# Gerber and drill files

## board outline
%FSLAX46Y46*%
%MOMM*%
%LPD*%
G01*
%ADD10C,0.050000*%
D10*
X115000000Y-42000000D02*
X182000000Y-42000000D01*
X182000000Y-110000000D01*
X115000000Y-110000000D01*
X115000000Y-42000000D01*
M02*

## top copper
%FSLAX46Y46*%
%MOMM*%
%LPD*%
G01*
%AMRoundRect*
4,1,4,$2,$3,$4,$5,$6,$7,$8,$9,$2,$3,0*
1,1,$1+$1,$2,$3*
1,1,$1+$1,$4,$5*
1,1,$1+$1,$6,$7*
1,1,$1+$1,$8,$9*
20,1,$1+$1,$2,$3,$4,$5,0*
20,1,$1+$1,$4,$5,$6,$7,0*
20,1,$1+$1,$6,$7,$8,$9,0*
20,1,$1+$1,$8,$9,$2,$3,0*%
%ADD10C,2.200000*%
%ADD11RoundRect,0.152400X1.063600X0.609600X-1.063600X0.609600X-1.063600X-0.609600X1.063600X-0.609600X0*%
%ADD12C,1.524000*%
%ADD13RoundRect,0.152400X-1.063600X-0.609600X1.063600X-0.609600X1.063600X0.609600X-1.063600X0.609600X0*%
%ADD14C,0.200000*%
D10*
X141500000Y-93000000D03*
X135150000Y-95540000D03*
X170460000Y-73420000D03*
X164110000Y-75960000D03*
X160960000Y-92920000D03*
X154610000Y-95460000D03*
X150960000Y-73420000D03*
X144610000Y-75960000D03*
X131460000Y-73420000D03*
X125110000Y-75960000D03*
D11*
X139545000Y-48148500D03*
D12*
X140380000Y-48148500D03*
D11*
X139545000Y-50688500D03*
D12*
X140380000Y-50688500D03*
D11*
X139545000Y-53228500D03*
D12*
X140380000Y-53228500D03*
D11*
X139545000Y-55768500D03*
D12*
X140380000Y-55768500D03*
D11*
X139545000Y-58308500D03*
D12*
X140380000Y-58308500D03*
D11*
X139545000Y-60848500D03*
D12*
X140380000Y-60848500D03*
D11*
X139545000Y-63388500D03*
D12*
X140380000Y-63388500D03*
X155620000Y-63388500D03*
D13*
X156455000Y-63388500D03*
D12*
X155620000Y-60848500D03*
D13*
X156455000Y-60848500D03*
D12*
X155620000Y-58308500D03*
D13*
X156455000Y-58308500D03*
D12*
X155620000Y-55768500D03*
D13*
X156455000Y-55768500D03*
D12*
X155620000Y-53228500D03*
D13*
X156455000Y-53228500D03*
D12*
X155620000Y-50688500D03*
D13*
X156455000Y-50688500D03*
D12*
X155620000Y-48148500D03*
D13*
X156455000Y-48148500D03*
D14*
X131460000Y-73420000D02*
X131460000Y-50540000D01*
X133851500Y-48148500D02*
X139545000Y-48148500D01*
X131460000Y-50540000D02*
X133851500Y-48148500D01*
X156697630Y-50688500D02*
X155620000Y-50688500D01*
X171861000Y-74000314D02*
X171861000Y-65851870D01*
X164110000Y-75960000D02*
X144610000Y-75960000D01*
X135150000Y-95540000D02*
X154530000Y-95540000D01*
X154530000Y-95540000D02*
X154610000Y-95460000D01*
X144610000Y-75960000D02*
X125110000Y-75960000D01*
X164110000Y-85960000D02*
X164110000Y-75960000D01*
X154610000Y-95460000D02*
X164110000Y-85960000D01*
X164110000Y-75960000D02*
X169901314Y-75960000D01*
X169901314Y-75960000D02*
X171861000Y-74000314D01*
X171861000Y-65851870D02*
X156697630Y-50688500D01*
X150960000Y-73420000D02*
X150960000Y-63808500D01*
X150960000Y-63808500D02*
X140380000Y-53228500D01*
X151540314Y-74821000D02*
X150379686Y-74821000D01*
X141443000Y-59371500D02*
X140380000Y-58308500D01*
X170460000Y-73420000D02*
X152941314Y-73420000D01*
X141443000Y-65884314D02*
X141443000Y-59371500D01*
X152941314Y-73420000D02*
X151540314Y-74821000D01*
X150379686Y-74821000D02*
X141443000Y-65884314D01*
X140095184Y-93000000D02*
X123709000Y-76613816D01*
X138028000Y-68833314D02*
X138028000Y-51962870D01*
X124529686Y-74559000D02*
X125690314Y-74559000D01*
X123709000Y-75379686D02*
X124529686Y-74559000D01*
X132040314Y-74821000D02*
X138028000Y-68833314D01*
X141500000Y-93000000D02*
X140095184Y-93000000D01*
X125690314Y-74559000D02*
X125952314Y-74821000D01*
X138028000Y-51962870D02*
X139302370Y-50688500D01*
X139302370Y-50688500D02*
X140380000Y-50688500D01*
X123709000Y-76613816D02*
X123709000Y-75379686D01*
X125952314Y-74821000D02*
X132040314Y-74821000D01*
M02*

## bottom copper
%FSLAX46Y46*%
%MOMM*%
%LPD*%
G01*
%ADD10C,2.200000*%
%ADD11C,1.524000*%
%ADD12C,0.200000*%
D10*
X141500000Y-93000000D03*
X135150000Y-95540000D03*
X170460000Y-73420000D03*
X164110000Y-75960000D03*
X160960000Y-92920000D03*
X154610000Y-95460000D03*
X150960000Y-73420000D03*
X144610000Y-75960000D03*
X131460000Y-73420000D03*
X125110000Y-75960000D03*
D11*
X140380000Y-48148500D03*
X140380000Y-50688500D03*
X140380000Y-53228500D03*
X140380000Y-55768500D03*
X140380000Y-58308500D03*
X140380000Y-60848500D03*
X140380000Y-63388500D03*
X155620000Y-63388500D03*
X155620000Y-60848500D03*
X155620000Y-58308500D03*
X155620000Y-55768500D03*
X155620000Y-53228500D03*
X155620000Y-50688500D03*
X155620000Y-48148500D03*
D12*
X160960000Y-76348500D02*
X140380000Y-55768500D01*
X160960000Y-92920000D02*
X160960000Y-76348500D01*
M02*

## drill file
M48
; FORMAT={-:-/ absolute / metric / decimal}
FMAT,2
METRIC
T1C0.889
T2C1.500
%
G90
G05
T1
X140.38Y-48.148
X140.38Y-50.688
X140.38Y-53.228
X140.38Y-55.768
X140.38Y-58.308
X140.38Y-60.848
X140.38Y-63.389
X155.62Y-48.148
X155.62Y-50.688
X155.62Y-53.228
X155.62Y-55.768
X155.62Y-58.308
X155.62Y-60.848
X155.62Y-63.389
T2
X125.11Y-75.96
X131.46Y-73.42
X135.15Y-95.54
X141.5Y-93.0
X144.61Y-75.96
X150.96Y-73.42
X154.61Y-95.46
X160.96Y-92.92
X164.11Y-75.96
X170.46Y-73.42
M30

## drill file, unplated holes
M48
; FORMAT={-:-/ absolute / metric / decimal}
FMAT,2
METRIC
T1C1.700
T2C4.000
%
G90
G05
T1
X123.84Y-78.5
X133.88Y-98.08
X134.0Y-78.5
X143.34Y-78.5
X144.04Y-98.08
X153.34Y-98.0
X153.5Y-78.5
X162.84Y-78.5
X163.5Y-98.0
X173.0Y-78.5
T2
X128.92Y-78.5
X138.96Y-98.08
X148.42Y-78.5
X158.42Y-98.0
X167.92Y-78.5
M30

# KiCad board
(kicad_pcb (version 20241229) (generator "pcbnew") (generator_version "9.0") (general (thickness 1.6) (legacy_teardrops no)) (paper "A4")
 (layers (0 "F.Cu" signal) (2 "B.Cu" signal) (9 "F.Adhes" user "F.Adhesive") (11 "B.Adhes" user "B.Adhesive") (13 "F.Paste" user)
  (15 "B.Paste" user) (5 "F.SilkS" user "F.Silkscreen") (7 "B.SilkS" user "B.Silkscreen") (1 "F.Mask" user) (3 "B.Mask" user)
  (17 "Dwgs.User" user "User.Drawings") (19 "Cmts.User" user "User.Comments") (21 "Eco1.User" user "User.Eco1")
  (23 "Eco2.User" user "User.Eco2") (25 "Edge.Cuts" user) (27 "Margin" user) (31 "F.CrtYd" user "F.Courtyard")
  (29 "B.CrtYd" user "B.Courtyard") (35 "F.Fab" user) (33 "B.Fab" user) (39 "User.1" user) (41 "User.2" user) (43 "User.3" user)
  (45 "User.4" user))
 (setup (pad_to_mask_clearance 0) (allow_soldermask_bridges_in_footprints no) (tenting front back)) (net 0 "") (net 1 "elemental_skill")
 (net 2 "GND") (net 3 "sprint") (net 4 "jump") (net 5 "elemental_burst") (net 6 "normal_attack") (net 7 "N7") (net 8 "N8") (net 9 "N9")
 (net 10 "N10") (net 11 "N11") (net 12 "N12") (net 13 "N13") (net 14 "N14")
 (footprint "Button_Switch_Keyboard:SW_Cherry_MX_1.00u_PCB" (layer "F.Cu") (at 141.5 93)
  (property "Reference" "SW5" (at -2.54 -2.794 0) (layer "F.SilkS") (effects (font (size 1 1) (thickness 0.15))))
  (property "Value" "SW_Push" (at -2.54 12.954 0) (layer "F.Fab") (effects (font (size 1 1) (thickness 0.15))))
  (pad "" np_thru_hole circle (at -7.62 5.08) (size 1.7 1.7) (drill 1.7) (layers "*.Cu" "*.Mask"))
  (pad "" np_thru_hole circle (at -2.54 5.08) (size 4 4) (drill 4) (layers "*.Cu" "*.Mask"))
  (pad "" np_thru_hole circle (at 2.54 5.08) (size 1.7 1.7) (drill 1.7) (layers "*.Cu" "*.Mask"))
  (pad "1" thru_hole circle (at 0 0) (size 2.2 2.2) (drill 1.5) (layers "*.Cu" "*.Mask") (remove_unused_layers no) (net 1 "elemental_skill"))
  (pad "2" thru_hole circle (at -6.35 2.54) (size 2.2 2.2) (drill 1.5) (layers "*.Cu" "*.Mask") (remove_unused_layers no) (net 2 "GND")))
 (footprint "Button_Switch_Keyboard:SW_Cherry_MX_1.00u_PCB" (layer "F.Cu") (at 170.46 73.42)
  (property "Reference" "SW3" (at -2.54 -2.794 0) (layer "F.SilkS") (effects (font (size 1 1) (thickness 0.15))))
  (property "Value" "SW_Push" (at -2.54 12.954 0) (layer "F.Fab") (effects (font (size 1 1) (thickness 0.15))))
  (pad "" np_thru_hole circle (at -7.62 5.08) (size 1.7 1.7) (drill 1.7) (layers "*.Cu" "*.Mask"))
  (pad "" np_thru_hole circle (at -2.54 5.08) (size 4 4) (drill 4) (layers "*.Cu" "*.Mask"))
  (pad "" np_thru_hole circle (at 2.54 5.08) (size 1.7 1.7) (drill 1.7) (layers "*.Cu" "*.Mask"))
  (pad "1" thru_hole circle (at 0 0) (size 2.2 2.2) (drill 1.5) (layers "*.Cu" "*.Mask") (remove_unused_layers no) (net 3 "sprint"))
  (pad "2" thru_hole circle (at -6.35 2.54) (size 2.2 2.2) (drill 1.5) (layers "*.Cu" "*.Mask") (remove_unused_layers no) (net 2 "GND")))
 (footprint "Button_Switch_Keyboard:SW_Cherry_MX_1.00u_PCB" (layer "F.Cu") (at 160.96 92.92)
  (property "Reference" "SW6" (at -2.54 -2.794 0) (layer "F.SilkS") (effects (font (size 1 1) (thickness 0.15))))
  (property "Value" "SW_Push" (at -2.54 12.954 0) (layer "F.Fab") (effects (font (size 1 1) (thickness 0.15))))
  (pad "" np_thru_hole circle (at -7.62 5.08) (size 1.7 1.7) (drill 1.7) (layers "*.Cu" "*.Mask"))
  (pad "" np_thru_hole circle (at -2.54 5.08) (size 4 4) (drill 4) (layers "*.Cu" "*.Mask"))
  (pad "" np_thru_hole circle (at 2.54 5.08) (size 1.7 1.7) (drill 1.7) (layers "*.Cu" "*.Mask"))
  (pad "1" thru_hole circle (at 0 0) (size 2.2 2.2) (drill 1.5) (layers "*.Cu" "*.Mask") (remove_unused_layers no) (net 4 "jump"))
  (pad "2" thru_hole circle (at -6.35 2.54) (size 2.2 2.2) (drill 1.5) (layers "*.Cu" "*.Mask") (remove_unused_layers no) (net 2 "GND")))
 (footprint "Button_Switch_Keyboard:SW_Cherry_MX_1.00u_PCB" (layer "F.Cu") (at 150.96 73.42)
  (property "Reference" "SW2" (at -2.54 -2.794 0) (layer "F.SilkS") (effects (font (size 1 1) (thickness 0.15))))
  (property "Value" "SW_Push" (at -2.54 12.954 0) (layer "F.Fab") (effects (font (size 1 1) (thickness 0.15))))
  (pad "" np_thru_hole circle (at -7.62 5.08) (size 1.7 1.7) (drill 1.7) (layers "*.Cu" "*.Mask"))
  (pad "" np_thru_hole circle (at -2.54 5.08) (size 4 4) (drill 4) (layers "*.Cu" "*.Mask"))
  (pad "" np_thru_hole circle (at 2.54 5.08) (size 1.7 1.7) (drill 1.7) (layers "*.Cu" "*.Mask"))
  (pad "1" thru_hole circle (at 0 0) (size 2.2 2.2) (drill 1.5) (layers "*.Cu" "*.Mask") (remove_unused_layers no) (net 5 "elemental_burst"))
  (pad "2" thru_hole circle (at -6.35 2.54) (size 2.2 2.2) (drill 1.5) (layers "*.Cu" "*.Mask") (remove_unused_layers no) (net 2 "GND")))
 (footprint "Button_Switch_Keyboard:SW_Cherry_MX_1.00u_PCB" (layer "F.Cu") (at 131.46 73.42)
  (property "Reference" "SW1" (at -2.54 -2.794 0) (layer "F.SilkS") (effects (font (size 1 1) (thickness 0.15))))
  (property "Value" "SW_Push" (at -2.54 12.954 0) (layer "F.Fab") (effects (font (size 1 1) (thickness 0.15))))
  (pad "" np_thru_hole circle (at -7.62 5.08) (size 1.7 1.7) (drill 1.7) (layers "*.Cu" "*.Mask"))
  (pad "" np_thru_hole circle (at -2.54 5.08) (size 4 4) (drill 4) (layers "*.Cu" "*.Mask"))
  (pad "" np_thru_hole circle (at 2.54 5.08) (size 1.7 1.7) (drill 1.7) (layers "*.Cu" "*.Mask"))
  (pad "1" thru_hole circle (at 0 0) (size 2.2 2.2) (drill 1.5) (layers "*.Cu" "*.Mask") (remove_unused_layers no) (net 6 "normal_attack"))
  (pad "2" thru_hole circle (at -6.35 2.54) (size 2.2 2.2) (drill 1.5) (layers "*.Cu" "*.Mask") (remove_unused_layers no) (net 2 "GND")))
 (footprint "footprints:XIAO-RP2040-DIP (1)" (layer "F.Cu") (at 148 55.7685)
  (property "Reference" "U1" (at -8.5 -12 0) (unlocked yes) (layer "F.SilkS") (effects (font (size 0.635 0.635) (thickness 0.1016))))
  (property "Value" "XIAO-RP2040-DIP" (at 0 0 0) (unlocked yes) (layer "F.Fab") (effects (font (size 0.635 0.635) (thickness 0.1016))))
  (pad "1" smd roundrect (at -8.455 -7.62 180) (size 2.432 1.524) (layers "F.Cu" "F.Mask") (roundrect_rratio 0.1) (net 6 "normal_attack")
   (thermal_bridge_angle 45))
  (pad "1" thru_hole circle (at -7.62 -7.62 180) (size 1.524 1.524) (drill 0.889) (layers "*.Cu" "*.Mask") (remove_unused_layers no)
   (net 6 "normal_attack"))
  (pad "2" smd roundrect (at -8.455 -5.08 180) (size 2.432 1.524) (layers "F.Cu" "F.Mask") (roundrect_rratio 0.1) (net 1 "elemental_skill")
   (thermal_bridge_angle 45))
  (pad "2" thru_hole circle (at -7.62 -5.08 180) (size 1.524 1.524) (drill 0.889) (layers "*.Cu" "*.Mask") (remove_unused_layers no)
   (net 1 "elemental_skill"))
  (pad "3" smd roundrect (at -8.455 -2.54 180) (size 2.432 1.524) (layers "F.Cu" "F.Mask") (roundrect_rratio 0.1) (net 5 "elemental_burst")
   (thermal_bridge_angle 45))
  (pad "3" thru_hole circle (at -7.62 -2.54 180) (size 1.524 1.524) (drill 0.889) (layers "*.Cu" "*.Mask") (remove_unused_layers no)
   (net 5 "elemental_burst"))
  (pad "4" smd roundrect (at -8.455 0 180) (size 2.432 1.524) (layers "F.Cu" "F.Mask") (roundrect_rratio 0.1) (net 4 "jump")
   (thermal_bridge_angle 45))
  (pad "4" thru_hole circle (at -7.62 0 180) (size 1.524 1.524) (drill 0.889) (layers "*.Cu" "*.Mask") (remove_unused_layers no)
   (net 4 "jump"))
  (pad "5" smd roundrect (at -8.455 2.54 180) (size 2.432 1.524) (layers "F.Cu" "F.Mask") (roundrect_rratio 0.1) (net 3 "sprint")
   (thermal_bridge_angle 45))
  (pad "5" thru_hole circle (at -7.62 2.54 180) (size 1.524 1.524) (drill 0.889) (layers "*.Cu" "*.Mask") (remove_unused_layers no)
   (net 3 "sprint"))
  (pad "6" smd roundrect (at -8.455 5.08 180) (size 2.432 1.524) (layers "F.Cu" "F.Mask") (roundrect_rratio 0.1) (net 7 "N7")
   (thermal_bridge_angle 45))
  (pad "6" thru_hole circle (at -7.62 5.08 180) (size 1.524 1.524) (drill 0.889) (layers "*.Cu" "*.Mask") (remove_unused_layers no)
   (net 7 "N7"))
  (pad "7" smd roundrect (at -8.455 7.62 180) (size 2.432 1.524) (layers "F.Cu" "F.Mask") (roundrect_rratio 0.1) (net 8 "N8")
   (thermal_bridge_angle 45))
  (pad "7" thru_hole circle (at -7.62 7.62 180) (size 1.524 1.524) (drill 0.889) (layers "*.Cu" "*.Mask") (remove_unused_layers no)
   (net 8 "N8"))
  (pad "8" thru_hole circle (at 7.62 7.62) (size 1.524 1.524) (drill 0.889) (layers "*.Cu" "*.Mask") (remove_unused_layers no) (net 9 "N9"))
  (pad "8" smd roundrect (at 8.455 7.62) (size 2.432 1.524) (layers "F.Cu" "F.Mask") (roundrect_rratio 0.1) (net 9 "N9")
   (thermal_bridge_angle 45))
  (pad "9" thru_hole circle (at 7.62 5.08) (size 1.524 1.524) (drill 0.889) (layers "*.Cu" "*.Mask") (remove_unused_layers no)
   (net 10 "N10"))
  (pad "9" smd roundrect (at 8.455 5.08) (size 2.432 1.524) (layers "F.Cu" "F.Mask") (roundrect_rratio 0.1) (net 10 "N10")
   (thermal_bridge_angle 45))
  (pad "10" thru_hole circle (at 7.62 2.54) (size 1.524 1.524) (drill 0.889) (layers "*.Cu" "*.Mask") (remove_unused_layers no)
   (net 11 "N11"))
  (pad "10" smd roundrect (at 8.455 2.54) (size 2.432 1.524) (layers "F.Cu" "F.Mask") (roundrect_rratio 0.1) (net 11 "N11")
   (thermal_bridge_angle 45))
  (pad "11" thru_hole circle (at 7.62 0) (size 1.524 1.524) (drill 0.889) (layers "*.Cu" "*.Mask") (remove_unused_layers no) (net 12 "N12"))
  (pad "11" smd roundrect (at 8.455 0) (size 2.432 1.524) (layers "F.Cu" "F.Mask") (roundrect_rratio 0.1) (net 12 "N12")
   (thermal_bridge_angle 45))
  (pad "12" thru_hole circle (at 7.62 -2.54) (size 1.524 1.524) (drill 0.889) (layers "*.Cu" "*.Mask") (remove_unused_layers no)
   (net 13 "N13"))
  (pad "12" smd roundrect (at 8.455 -2.54) (size 2.432 1.524) (layers "F.Cu" "F.Mask") (roundrect_rratio 0.1) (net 13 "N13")
   (thermal_bridge_angle 45))
  (pad "13" thru_hole circle (at 7.62 -5.08) (size 1.524 1.524) (drill 0.889) (layers "*.Cu" "*.Mask") (remove_unused_layers no)
   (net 2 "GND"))
  (pad "13" smd roundrect (at 8.455 -5.08) (size 2.432 1.524) (layers "F.Cu" "F.Mask") (roundrect_rratio 0.1) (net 2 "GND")
   (thermal_bridge_angle 45))
  (pad "14" thru_hole circle (at 7.62 -7.62) (size 1.524 1.524) (drill 0.889) (layers "*.Cu" "*.Mask") (remove_unused_layers no)
   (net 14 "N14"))
  (pad "14" smd roundrect (at 8.455 -7.62) (size 2.432 1.524) (layers "F.Cu" "F.Mask") (roundrect_rratio 0.1) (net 14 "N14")
   (thermal_bridge_angle 45)))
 (gr_rect (start 115 42) (end 182 110) (stroke (width 0.05) (type solid)) (fill no) (layer "Edge.Cuts"))
 (segment (start 131.46 73.42) (end 131.46 50.54) (width 0.2) (layer "F.Cu") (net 6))
 (segment (start 133.8515 48.1485) (end 139.545 48.1485) (width 0.2) (layer "F.Cu") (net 6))
 (segment (start 131.46 50.54) (end 133.8515 48.1485) (width 0.2) (layer "F.Cu") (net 6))
 (segment (start 156.69763 50.6885) (end 155.62 50.6885) (width 0.2) (layer "F.Cu") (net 2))
 (segment (start 171.861 74.000314) (end 171.861 65.85187) (width 0.2) (layer "F.Cu") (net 2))
 (segment (start 164.11 75.96) (end 144.61 75.96) (width 0.2) (layer "F.Cu") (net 2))
 (segment (start 135.15 95.54) (end 154.53 95.54) (width 0.2) (layer "F.Cu") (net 2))
 (segment (start 154.53 95.54) (end 154.61 95.46) (width 0.2) (layer "F.Cu") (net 2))
 (segment (start 144.61 75.96) (end 125.11 75.96) (width 0.2) (layer "F.Cu") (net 2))
 (segment (start 164.11 85.96) (end 164.11 75.96) (width 0.2) (layer "F.Cu") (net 2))
 (segment (start 154.61 95.46) (end 164.11 85.96) (width 0.2) (layer "F.Cu") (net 2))
 (segment (start 164.11 75.96) (end 169.901314 75.96) (width 0.2) (layer "F.Cu") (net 2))
 (segment (start 169.901314 75.96) (end 171.861 74.000314) (width 0.2) (layer "F.Cu") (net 2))
 (segment (start 171.861 65.85187) (end 156.69763 50.6885) (width 0.2) (layer "F.Cu") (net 2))
 (segment (start 150.96 73.42) (end 150.96 63.8085) (width 0.2) (layer "F.Cu") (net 5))
 (segment (start 150.96 63.8085) (end 140.38 53.2285) (width 0.2) (layer "F.Cu") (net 5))
 (segment (start 151.540314 74.821) (end 150.379686 74.821) (width 0.2) (layer "F.Cu") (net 3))
 (segment (start 141.443 59.3715) (end 140.38 58.3085) (width 0.2) (layer "F.Cu") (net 3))
 (segment (start 170.46 73.42) (end 152.941314 73.42) (width 0.2) (layer "F.Cu") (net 3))
 (segment (start 141.443 65.884314) (end 141.443 59.3715) (width 0.2) (layer "F.Cu") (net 3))
 (segment (start 152.941314 73.42) (end 151.540314 74.821) (width 0.2) (layer "F.Cu") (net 3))
 (segment (start 150.379686 74.821) (end 141.443 65.884314) (width 0.2) (layer "F.Cu") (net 3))
 (segment (start 140.095184 93) (end 123.709 76.613816) (width 0.2) (layer "F.Cu") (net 1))
 (segment (start 138.028 68.833314) (end 138.028 51.96287) (width 0.2) (layer "F.Cu") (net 1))
 (segment (start 124.529686 74.559) (end 125.690314 74.559) (width 0.2) (layer "F.Cu") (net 1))
 (segment (start 123.709 75.379686) (end 124.529686 74.559) (width 0.2) (layer "F.Cu") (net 1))
 (segment (start 132.040314 74.821) (end 138.028 68.833314) (width 0.2) (layer "F.Cu") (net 1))
 (segment (start 141.5 93) (end 140.095184 93) (width 0.2) (layer "F.Cu") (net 1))
 (segment (start 125.690314 74.559) (end 125.952314 74.821) (width 0.2) (layer "F.Cu") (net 1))
 (segment (start 138.028 51.96287) (end 139.30237 50.6885) (width 0.2) (layer "F.Cu") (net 1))
 (segment (start 139.30237 50.6885) (end 140.38 50.6885) (width 0.2) (layer "F.Cu") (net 1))
 (segment (start 123.709 76.613816) (end 123.709 75.379686) (width 0.2) (layer "F.Cu") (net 1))
 (segment (start 125.952314 74.821) (end 132.040314 74.821) (width 0.2) (layer "F.Cu") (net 1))
 (segment (start 160.96 76.3485) (end 140.38 55.7685) (width 0.2) (layer "B.Cu") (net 4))
 (segment (start 160.96 92.92) (end 160.96 76.3485) (width 0.2) (layer "B.Cu") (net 4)))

